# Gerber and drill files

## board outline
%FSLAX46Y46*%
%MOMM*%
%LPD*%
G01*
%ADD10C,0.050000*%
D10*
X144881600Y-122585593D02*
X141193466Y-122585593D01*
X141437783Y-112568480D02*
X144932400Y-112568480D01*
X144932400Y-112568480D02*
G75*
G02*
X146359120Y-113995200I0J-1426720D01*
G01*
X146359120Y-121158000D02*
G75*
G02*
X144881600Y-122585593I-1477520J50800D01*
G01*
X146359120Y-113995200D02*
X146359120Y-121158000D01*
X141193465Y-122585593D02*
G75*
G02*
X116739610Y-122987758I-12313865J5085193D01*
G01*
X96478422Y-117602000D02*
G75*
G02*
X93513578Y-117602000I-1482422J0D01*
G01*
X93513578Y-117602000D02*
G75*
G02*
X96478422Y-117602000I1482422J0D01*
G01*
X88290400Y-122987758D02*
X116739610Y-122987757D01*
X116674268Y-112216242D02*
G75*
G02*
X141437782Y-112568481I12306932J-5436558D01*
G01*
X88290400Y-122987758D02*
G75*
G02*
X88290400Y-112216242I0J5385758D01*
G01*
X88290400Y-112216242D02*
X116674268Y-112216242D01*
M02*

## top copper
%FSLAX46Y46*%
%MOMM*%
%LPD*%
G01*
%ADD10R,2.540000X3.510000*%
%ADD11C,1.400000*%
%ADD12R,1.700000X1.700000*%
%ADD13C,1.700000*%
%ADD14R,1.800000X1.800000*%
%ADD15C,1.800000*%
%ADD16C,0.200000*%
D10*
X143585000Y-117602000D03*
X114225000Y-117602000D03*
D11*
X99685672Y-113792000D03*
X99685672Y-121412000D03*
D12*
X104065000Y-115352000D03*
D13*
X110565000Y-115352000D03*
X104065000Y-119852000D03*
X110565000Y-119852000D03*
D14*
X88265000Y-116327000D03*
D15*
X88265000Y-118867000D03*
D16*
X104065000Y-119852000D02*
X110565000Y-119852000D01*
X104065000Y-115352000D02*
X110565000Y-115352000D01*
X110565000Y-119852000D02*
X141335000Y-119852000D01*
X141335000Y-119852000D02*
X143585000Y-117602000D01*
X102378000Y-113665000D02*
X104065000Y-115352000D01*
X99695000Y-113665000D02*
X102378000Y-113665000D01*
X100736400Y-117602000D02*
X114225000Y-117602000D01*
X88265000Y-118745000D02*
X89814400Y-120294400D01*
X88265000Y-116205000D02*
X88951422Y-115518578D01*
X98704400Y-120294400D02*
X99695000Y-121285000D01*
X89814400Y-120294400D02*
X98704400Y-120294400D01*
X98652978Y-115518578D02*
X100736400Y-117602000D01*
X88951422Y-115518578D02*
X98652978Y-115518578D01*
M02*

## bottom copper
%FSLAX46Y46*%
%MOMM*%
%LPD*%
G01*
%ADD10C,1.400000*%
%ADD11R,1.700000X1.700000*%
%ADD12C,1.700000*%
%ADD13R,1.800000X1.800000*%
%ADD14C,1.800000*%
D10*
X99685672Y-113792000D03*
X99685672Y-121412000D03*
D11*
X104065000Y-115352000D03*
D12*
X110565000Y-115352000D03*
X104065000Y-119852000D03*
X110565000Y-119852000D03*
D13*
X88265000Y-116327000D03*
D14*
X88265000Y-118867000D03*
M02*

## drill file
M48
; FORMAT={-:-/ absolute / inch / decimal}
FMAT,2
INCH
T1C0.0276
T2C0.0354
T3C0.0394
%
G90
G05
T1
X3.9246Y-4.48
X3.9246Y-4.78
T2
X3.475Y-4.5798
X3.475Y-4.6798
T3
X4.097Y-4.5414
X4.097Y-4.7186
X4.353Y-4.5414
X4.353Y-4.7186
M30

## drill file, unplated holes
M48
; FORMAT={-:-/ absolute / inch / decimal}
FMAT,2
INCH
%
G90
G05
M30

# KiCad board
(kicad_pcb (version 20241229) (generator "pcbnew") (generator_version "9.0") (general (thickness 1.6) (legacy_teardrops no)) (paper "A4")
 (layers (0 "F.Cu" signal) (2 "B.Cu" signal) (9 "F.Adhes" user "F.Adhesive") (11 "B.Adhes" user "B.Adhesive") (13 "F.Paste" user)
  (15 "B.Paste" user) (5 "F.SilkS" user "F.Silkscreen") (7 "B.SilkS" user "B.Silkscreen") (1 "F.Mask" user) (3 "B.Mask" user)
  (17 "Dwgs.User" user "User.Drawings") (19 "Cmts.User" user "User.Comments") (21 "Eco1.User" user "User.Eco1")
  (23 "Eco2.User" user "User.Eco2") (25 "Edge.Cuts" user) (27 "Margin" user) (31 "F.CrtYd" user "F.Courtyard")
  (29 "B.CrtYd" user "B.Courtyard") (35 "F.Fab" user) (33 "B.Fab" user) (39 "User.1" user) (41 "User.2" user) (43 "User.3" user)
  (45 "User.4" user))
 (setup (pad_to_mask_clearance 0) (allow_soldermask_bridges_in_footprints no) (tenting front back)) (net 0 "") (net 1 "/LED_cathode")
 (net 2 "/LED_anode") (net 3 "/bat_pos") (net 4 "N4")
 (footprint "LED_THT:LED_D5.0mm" (layer "F.Cu") (at 88.265 116.327 -90)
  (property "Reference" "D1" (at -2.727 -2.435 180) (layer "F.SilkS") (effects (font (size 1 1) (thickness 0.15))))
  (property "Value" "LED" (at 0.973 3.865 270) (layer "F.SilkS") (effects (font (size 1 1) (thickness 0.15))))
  (pad "1" thru_hole rect (at 0 0 270) (size 1.8 1.8) (drill 0.9) (layers "*.Cu" "*.Mask") (remove_unused_layers no) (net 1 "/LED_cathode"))
  (pad "2" thru_hole circle (at 2.54 0 270) (size 1.8 1.8) (drill 0.9) (layers "*.Cu" "*.Mask") (remove_unused_layers no)
   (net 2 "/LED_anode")))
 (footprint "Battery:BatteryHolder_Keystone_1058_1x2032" (layer "F.Cu") (at 128.905 117.602 180)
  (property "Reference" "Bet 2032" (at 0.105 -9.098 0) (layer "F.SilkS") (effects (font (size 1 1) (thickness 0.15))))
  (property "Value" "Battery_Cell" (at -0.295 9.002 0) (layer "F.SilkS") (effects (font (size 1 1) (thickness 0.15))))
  (pad "1" smd rect (at -14.68 0 180) (size 2.54 3.51) (layers "F.Cu" "F.Mask" "F.Paste") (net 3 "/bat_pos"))
  (pad "2" smd rect (at 14.68 0 180) (size 2.54 3.51) (layers "F.Cu" "F.Mask" "F.Paste") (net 1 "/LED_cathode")))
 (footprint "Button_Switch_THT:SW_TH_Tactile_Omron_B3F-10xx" (layer "F.Cu") (at 104.065 115.352)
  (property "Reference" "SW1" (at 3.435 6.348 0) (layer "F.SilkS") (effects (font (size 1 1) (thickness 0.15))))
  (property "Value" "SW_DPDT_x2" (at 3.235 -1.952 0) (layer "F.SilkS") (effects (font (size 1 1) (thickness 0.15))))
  (pad "1" thru_hole rect (at 0 0) (size 1.7 1.7) (drill 1) (layers "*.Cu" "*.Mask") (remove_unused_layers no) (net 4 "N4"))
  (pad "1" thru_hole circle (at 6.5 0) (size 1.7 1.7) (drill 1) (layers "*.Cu" "*.Mask") (remove_unused_layers no) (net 4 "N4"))
  (pad "2" thru_hole circle (at 0 4.5) (size 1.7 1.7) (drill 1) (layers "*.Cu" "*.Mask") (remove_unused_layers no) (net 3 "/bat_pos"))
  (pad "2" thru_hole circle (at 6.5 4.5) (size 1.7 1.7) (drill 1) (layers "*.Cu" "*.Mask") (remove_unused_layers no) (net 3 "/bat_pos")))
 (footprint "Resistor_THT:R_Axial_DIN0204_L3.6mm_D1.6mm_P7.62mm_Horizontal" (layer "F.Cu") (at 99.6857 113.792 -90)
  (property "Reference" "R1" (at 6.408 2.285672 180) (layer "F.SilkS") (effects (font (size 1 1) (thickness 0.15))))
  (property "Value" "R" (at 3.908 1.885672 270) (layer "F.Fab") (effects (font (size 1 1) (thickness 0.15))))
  (pad "1" thru_hole circle (at 0 0 270) (size 1.4 1.4) (drill 0.7) (layers "*.Cu" "*.Mask") (remove_unused_layers no) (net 4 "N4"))
  (pad "2" thru_hole circle (at 7.62 0 270) (size 1.4 1.4) (drill 0.7) (layers "*.Cu" "*.Mask") (remove_unused_layers no)
   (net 2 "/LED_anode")))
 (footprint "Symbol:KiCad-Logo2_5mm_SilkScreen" (layer "B.Cu") (at 129.54 114.5 180)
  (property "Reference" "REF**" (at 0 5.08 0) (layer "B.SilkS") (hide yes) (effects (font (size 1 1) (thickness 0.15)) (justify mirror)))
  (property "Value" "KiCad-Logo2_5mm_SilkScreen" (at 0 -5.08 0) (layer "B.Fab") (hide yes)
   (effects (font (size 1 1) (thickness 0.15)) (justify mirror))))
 (gr_line (start 88.2904 112.216242) (end 116.674268 112.216242) (stroke (width 0.05) (type default)) (locked yes) (layer "Edge.Cuts"))
 (gr_arc (start 88.2904 122.987758) (mid 82.904642 117.602) (end 88.2904 112.216242) (stroke (width 0.05) (type default)) (locked yes)
  (layer "Edge.Cuts"))
 (gr_circle (center 94.996 117.602) (end 96.012 118.6815) (stroke (width 0.05) (type default)) (fill no) (layer "Edge.Cuts"))
 (gr_line (start 88.2904 122.987758) (end 116.73961 122.987757) (stroke (width 0.05) (type default)) (locked yes) (layer "Edge.Cuts"))
 (gr_line (start 141.437783 112.56848) (end 144.9324 112.56848) (stroke (width 0.05) (type default)) (locked yes) (layer "Edge.Cuts"))
 (gr_arc (start 144.9324 112.56848) (mid 145.941243 112.986357) (end 146.35912 113.9952) (stroke (width 0.05) (type default)) (locked yes)
  (layer "Edge.Cuts"))
 (gr_line (start 144.8816 122.585593) (end 141.193466 122.585593) (stroke (width 0.05) (type default)) (locked yes) (layer "Edge.Cuts"))
 (gr_line (start 146.35912 113.9952) (end 146.35912 121.158) (stroke (width 0.05) (type default)) (locked yes) (layer "Edge.Cuts"))
 (gr_arc (start 141.193465 122.585593) (mid 129.098671 130.821153) (end 116.73961 122.987758) (stroke (width 0.05) (type default))
  (locked yes) (layer "Edge.Cuts"))
 (gr_arc (start 146.35912 121.158) (mid 145.908864 122.170391) (end 144.8816 122.585593) (stroke (width 0.05) (type default)) (locked yes)
  (layer "Edge.Cuts"))
 (gr_arc (start 116.674268 112.216242) (mid 129.172555 104.199915) (end 141.437782 112.568481) (stroke (width 0.05) (type default))
  (locked yes) (layer "Edge.Cuts"))
 (segment (start 110.565 119.852) (end 104.065 119.852) (width 0.2) (layer "F.Cu") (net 3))
 (segment (start 104.065 119.852) (end 141.335 119.852) (width 0.2) (layer "F.Cu") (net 3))
 (segment (start 141.335 119.852) (end 143.585 117.602) (width 0.2) (layer "F.Cu") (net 3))
 (segment (start 88.9514 115.519) (end 98.653 115.519) (width 0.2) (layer "F.Cu") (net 1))
 (segment (start 98.653 115.519) (end 100.736 117.602) (width 0.2) (layer "F.Cu") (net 1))
 (segment (start 88.265 116.205) (end 88.9514 115.519) (width 0.2) (layer "F.Cu") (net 1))
 (segment (start 88.265 116.327) (end 88.265 116.205) (width 0.2) (layer "F.Cu") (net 1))
 (segment (start 100.736 117.602) (end 114.225 117.602) (width 0.2) (layer "F.Cu") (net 1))
 (segment (start 99.695 121.4027) (end 99.695 121.285) (width 0.2) (layer "F.Cu") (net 2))
 (segment (start 99.6857 121.412) (end 99.695 121.4027) (width 0.2) (layer "F.Cu") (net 2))
 (segment (start 89.0397 119.5195) (end 88.9175 119.5195) (width 0.2) (layer "F.Cu") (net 2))
 (segment (start 89.0397 119.5195) (end 89.8144 120.294) (width 0.2) (layer "F.Cu") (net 2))
 (segment (start 88.265 118.745) (end 89.0397 119.5195) (width 0.2) (layer "F.Cu") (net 2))
 (segment (start 88.9175 119.5195) (end 88.265 118.867) (width 0.2) (layer "F.Cu") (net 2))
 (segment (start 98.7044 120.294) (end 99.695 121.285) (width 0.2) (layer "F.Cu") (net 2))
 (segment (start 89.8144 120.294) (end 98.7044 120.294) (width 0.2) (layer "F.Cu") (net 2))
 (segment (start 99.6857 113.792) (end 99.695 113.7827) (width 0.2) (layer "F.Cu") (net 4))
 (segment (start 104.065 115.352) (end 110.565 115.352) (width 0.2) (layer "F.Cu") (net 4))
 (segment (start 102.378 113.665) (end 104.065 115.352) (width 0.2) (layer "F.Cu") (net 4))
 (segment (start 99.695 113.7827) (end 99.695 113.665) (width 0.2) (layer "F.Cu") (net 4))
 (segment (start 99.695 113.665) (end 102.378 113.665) (width 0.2) (layer "F.Cu") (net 4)))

